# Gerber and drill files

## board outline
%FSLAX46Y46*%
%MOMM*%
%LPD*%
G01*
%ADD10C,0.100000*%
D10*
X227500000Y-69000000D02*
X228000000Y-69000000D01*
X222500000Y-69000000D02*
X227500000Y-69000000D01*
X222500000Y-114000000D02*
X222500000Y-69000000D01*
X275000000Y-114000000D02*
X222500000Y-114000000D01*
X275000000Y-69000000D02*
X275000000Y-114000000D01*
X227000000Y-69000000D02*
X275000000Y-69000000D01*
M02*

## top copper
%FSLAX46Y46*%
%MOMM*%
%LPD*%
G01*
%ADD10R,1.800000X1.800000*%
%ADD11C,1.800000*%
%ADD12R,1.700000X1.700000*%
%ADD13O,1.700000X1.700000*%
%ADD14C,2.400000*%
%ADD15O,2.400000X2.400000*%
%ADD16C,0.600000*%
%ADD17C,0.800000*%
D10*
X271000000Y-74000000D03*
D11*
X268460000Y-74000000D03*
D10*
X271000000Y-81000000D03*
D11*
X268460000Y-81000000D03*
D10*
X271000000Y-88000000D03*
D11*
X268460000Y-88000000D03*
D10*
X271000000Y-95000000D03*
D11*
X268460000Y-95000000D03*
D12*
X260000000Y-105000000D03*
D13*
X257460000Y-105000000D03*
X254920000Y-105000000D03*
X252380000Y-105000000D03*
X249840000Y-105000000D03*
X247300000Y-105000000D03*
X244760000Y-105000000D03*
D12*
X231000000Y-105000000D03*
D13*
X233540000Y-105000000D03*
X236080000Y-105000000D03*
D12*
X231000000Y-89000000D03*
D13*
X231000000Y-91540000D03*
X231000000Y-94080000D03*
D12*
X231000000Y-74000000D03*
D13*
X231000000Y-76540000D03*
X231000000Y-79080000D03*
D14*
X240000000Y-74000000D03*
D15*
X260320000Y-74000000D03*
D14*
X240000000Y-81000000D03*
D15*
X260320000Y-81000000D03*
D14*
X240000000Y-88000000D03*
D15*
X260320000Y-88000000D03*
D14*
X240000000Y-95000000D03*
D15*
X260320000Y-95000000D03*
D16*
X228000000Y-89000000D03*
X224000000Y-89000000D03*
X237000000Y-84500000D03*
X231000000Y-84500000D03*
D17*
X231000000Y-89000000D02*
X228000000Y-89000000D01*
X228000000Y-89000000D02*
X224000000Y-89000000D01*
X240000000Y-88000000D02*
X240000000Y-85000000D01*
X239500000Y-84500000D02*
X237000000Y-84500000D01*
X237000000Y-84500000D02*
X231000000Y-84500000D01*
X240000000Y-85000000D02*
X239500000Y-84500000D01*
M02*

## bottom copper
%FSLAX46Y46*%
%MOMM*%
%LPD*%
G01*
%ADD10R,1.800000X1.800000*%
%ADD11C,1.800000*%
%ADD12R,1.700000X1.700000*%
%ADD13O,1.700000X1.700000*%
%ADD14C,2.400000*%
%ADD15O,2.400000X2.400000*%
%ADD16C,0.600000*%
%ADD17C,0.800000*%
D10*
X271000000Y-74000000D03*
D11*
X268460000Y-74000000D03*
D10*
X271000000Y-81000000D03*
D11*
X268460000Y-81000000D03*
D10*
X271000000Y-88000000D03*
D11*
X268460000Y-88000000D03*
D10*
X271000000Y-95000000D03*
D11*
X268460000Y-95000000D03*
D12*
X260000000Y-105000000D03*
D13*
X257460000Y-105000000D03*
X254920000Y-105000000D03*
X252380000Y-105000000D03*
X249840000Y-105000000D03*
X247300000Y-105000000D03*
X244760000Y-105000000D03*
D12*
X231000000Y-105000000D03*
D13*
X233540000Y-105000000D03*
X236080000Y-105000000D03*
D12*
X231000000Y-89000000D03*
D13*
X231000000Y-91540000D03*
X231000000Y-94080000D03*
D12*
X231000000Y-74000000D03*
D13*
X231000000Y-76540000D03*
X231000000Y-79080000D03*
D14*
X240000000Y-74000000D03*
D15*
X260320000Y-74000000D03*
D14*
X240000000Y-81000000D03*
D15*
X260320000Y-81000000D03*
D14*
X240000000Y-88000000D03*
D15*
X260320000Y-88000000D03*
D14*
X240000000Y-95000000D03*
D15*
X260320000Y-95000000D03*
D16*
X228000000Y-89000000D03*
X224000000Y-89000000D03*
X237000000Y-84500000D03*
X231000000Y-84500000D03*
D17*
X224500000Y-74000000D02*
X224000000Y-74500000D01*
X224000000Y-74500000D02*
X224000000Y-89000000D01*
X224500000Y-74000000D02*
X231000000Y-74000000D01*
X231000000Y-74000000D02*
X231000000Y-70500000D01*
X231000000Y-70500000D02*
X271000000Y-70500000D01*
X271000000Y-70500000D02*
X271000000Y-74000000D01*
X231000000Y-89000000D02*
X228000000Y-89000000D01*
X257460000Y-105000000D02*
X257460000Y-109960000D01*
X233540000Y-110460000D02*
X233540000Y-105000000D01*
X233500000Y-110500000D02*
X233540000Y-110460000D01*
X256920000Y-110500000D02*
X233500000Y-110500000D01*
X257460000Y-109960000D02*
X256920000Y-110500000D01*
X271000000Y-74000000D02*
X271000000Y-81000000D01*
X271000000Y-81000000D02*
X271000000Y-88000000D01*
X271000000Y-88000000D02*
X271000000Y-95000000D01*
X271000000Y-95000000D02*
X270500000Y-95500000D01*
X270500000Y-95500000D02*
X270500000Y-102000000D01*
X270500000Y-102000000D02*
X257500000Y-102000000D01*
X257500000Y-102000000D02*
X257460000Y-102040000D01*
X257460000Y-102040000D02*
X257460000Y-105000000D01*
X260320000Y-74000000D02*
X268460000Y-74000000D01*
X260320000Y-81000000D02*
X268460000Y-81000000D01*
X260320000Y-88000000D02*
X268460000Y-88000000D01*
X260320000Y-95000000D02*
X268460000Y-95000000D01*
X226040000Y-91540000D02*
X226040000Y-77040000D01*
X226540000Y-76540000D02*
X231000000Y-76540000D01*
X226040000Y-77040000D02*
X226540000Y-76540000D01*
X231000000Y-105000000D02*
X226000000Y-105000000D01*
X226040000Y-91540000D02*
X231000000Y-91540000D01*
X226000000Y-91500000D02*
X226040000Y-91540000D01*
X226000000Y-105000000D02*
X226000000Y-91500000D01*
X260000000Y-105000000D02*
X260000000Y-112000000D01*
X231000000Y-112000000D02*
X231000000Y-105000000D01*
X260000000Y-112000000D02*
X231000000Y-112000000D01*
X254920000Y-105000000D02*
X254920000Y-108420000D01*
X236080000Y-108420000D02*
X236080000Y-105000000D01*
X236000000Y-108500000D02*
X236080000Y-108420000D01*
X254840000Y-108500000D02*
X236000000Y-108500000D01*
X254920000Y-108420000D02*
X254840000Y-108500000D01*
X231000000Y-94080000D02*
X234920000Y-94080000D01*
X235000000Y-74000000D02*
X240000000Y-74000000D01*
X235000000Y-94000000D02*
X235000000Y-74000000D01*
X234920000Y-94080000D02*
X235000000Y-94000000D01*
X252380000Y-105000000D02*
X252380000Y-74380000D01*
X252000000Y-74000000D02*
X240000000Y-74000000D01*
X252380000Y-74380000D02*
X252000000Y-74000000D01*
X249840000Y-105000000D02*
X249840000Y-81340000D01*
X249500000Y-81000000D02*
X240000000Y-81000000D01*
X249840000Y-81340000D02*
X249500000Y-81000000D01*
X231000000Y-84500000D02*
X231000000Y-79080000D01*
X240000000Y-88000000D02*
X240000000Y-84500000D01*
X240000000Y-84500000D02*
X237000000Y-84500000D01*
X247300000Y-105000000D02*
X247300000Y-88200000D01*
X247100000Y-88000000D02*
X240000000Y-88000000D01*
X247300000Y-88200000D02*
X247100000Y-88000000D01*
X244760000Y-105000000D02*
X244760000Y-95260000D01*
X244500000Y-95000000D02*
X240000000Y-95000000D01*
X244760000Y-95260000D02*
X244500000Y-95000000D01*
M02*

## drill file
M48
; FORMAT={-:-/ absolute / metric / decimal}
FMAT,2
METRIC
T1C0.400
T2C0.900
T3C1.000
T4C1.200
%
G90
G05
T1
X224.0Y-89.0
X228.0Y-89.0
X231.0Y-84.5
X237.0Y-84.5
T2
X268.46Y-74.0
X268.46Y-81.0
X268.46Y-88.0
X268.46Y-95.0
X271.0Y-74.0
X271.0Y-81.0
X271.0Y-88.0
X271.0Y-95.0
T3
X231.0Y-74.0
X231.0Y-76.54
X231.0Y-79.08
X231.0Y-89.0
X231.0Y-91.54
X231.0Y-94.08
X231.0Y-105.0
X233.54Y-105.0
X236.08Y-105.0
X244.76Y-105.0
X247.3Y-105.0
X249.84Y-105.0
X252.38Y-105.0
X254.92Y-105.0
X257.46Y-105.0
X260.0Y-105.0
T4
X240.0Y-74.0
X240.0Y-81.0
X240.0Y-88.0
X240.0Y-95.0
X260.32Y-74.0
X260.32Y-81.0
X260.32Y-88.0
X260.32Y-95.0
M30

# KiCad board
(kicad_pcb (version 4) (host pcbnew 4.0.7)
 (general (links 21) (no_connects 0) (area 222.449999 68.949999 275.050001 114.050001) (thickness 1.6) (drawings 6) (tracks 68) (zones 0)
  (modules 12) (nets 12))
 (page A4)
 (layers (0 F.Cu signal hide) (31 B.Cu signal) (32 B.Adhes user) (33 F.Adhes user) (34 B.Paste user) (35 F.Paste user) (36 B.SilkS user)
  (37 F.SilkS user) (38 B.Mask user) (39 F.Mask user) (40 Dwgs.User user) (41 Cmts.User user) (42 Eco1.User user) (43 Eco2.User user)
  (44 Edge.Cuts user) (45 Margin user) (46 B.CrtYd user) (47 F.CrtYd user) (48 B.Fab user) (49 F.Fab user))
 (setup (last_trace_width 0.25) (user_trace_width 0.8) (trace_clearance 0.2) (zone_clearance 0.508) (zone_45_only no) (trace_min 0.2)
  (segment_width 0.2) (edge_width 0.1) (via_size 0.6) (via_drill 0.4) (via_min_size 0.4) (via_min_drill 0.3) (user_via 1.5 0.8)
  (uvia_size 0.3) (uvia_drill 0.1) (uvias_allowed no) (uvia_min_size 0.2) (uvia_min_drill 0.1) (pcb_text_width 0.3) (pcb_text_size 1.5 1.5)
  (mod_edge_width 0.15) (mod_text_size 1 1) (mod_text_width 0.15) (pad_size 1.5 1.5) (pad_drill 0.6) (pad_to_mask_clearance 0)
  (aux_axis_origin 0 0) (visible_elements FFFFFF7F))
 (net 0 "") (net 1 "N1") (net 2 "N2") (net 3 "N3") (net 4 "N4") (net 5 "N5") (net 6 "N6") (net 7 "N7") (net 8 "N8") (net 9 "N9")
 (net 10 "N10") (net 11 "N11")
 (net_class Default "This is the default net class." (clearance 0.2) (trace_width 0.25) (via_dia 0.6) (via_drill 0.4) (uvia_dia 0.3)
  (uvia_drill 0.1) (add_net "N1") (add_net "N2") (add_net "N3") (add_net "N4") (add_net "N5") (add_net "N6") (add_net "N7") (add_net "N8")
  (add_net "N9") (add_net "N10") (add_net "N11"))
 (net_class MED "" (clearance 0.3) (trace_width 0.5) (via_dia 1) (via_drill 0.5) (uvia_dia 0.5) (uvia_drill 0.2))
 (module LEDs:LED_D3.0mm (layer F.Cu) (at 271 74 180)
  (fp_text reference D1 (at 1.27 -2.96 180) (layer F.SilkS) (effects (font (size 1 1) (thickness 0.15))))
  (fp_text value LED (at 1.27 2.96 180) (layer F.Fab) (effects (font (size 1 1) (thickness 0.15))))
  (pad 1 thru_hole rect (at 0 0 180) (size 1.8 1.8) (drill 0.9) (layers *.Cu *.Mask) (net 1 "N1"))
  (pad 2 thru_hole circle (at 2.54 0 180) (size 1.8 1.8) (drill 0.9) (layers *.Cu *.Mask) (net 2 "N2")))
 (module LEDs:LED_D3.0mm (layer F.Cu) (at 271 81 180)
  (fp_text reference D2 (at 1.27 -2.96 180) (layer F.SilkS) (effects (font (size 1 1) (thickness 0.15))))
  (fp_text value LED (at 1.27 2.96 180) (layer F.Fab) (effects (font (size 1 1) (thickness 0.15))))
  (pad 1 thru_hole rect (at 0 0 180) (size 1.8 1.8) (drill 0.9) (layers *.Cu *.Mask) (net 1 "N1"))
  (pad 2 thru_hole circle (at 2.54 0 180) (size 1.8 1.8) (drill 0.9) (layers *.Cu *.Mask) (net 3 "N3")))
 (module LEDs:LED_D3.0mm (layer F.Cu) (at 271 88 180)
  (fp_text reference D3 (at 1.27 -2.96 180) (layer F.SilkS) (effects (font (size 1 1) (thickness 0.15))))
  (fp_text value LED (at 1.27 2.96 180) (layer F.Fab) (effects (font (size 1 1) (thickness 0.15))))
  (pad 1 thru_hole rect (at 0 0 180) (size 1.8 1.8) (drill 0.9) (layers *.Cu *.Mask) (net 1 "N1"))
  (pad 2 thru_hole circle (at 2.54 0 180) (size 1.8 1.8) (drill 0.9) (layers *.Cu *.Mask) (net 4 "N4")))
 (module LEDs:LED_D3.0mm (layer F.Cu) (at 271 95 180)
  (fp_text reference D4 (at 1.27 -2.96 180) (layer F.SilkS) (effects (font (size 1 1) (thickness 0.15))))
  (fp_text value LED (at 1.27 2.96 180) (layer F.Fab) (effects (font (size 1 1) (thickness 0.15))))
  (pad 1 thru_hole rect (at 0 0 180) (size 1.8 1.8) (drill 0.9) (layers *.Cu *.Mask) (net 1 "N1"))
  (pad 2 thru_hole circle (at 2.54 0 180) (size 1.8 1.8) (drill 0.9) (layers *.Cu *.Mask) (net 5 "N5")))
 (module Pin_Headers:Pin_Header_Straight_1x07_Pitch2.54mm (layer F.Cu) (at 260 105 270)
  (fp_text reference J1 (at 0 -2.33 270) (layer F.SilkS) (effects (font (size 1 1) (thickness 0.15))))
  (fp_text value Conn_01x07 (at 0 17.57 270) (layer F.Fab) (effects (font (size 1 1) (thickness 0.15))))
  (pad 1 thru_hole rect (at 0 0 270) (size 1.7 1.7) (drill 1) (layers *.Cu *.Mask) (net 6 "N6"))
  (pad 2 thru_hole oval (at 0 2.54 270) (size 1.7 1.7) (drill 1) (layers *.Cu *.Mask) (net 1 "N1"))
  (pad 3 thru_hole oval (at 0 5.08 270) (size 1.7 1.7) (drill 1) (layers *.Cu *.Mask) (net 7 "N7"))
  (pad 4 thru_hole oval (at 0 7.62 270) (size 1.7 1.7) (drill 1) (layers *.Cu *.Mask) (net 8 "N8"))
  (pad 5 thru_hole oval (at 0 10.16 270) (size 1.7 1.7) (drill 1) (layers *.Cu *.Mask) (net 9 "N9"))
  (pad 6 thru_hole oval (at 0 12.7 270) (size 1.7 1.7) (drill 1) (layers *.Cu *.Mask) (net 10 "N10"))
  (pad 7 thru_hole oval (at 0 15.24 270) (size 1.7 1.7) (drill 1) (layers *.Cu *.Mask) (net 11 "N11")))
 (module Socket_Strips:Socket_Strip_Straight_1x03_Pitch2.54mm (layer F.Cu) (at 231 105 90)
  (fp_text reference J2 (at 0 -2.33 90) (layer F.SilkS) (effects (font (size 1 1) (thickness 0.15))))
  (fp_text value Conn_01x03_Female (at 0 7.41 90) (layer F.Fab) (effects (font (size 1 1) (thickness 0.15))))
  (pad 1 thru_hole rect (at 0 0 90) (size 1.7 1.7) (drill 1) (layers *.Cu *.Mask) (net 6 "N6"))
  (pad 2 thru_hole oval (at 0 2.54 90) (size 1.7 1.7) (drill 1) (layers *.Cu *.Mask) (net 1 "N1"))
  (pad 3 thru_hole oval (at 0 5.08 90) (size 1.7 1.7) (drill 1) (layers *.Cu *.Mask) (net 7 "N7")))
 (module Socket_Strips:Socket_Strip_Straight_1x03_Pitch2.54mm (layer F.Cu) (at 231 89)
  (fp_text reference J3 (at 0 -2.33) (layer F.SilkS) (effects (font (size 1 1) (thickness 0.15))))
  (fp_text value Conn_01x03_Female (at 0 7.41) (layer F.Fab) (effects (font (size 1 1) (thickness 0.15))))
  (pad 1 thru_hole rect (at 0 0) (size 1.7 1.7) (drill 1) (layers *.Cu *.Mask) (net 1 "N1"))
  (pad 2 thru_hole oval (at 0 2.54) (size 1.7 1.7) (drill 1) (layers *.Cu *.Mask) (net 6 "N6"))
  (pad 3 thru_hole oval (at 0 5.08) (size 1.7 1.7) (drill 1) (layers *.Cu *.Mask) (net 8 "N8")))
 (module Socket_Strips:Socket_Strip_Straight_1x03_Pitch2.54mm (layer F.Cu) (at 231 74)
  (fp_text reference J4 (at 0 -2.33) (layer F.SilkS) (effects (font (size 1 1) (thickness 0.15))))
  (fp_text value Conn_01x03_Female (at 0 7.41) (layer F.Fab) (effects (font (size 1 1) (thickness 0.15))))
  (pad 1 thru_hole rect (at 0 0) (size 1.7 1.7) (drill 1) (layers *.Cu *.Mask) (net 1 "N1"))
  (pad 2 thru_hole oval (at 0 2.54) (size 1.7 1.7) (drill 1) (layers *.Cu *.Mask) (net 6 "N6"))
  (pad 3 thru_hole oval (at 0 5.08) (size 1.7 1.7) (drill 1) (layers *.Cu *.Mask) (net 10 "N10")))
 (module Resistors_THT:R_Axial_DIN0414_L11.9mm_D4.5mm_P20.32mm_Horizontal (layer F.Cu) (at 240 74)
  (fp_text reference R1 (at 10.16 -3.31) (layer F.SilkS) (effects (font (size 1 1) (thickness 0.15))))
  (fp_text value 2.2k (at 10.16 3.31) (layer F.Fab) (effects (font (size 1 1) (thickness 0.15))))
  (pad 1 thru_hole circle (at 0 0) (size 2.4 2.4) (drill 1.2) (layers *.Cu *.Mask) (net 8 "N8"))
  (pad 2 thru_hole oval (at 20.32 0) (size 2.4 2.4) (drill 1.2) (layers *.Cu *.Mask) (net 2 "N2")))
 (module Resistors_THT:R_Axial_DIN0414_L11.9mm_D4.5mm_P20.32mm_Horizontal (layer F.Cu) (at 240 81)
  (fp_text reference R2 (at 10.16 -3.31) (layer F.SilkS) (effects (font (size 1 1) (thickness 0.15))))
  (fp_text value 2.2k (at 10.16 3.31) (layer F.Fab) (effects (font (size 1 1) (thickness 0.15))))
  (pad 1 thru_hole circle (at 0 0) (size 2.4 2.4) (drill 1.2) (layers *.Cu *.Mask) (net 9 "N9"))
  (pad 2 thru_hole oval (at 20.32 0) (size 2.4 2.4) (drill 1.2) (layers *.Cu *.Mask) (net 3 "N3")))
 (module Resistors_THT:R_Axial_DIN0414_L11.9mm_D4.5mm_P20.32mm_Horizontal (layer F.Cu) (at 240 88)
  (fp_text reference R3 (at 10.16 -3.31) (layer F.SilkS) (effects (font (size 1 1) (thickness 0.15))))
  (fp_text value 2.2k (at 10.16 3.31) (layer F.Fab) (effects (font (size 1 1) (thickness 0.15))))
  (pad 1 thru_hole circle (at 0 0) (size 2.4 2.4) (drill 1.2) (layers *.Cu *.Mask) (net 10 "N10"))
  (pad 2 thru_hole oval (at 20.32 0) (size 2.4 2.4) (drill 1.2) (layers *.Cu *.Mask) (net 4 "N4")))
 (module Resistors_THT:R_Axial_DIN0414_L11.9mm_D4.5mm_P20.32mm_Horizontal (layer F.Cu) (at 240 95)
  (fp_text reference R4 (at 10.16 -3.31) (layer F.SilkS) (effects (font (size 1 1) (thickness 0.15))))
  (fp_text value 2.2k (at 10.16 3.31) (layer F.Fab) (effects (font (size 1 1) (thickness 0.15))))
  (pad 1 thru_hole circle (at 0 0) (size 2.4 2.4) (drill 1.2) (layers *.Cu *.Mask) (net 11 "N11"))
  (pad 2 thru_hole oval (at 20.32 0) (size 2.4 2.4) (drill 1.2) (layers *.Cu *.Mask) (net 5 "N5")))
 (gr_line (start 227.5 69) (end 228 69) (angle 90) (layer Edge.Cuts) (width 0.1))
 (gr_line (start 222.5 69) (end 227.5 69) (angle 90) (layer Edge.Cuts) (width 0.1))
 (gr_line (start 222.5 114) (end 222.5 69) (angle 90) (layer Edge.Cuts) (width 0.1))
 (gr_line (start 275 114) (end 222.5 114) (angle 90) (layer Edge.Cuts) (width 0.1))
 (gr_line (start 275 69) (end 275 114) (angle 90) (layer Edge.Cuts) (width 0.1))
 (gr_line (start 227 69) (end 275 69) (angle 90) (layer Edge.Cuts) (width 0.1))
 (via (at 228 89) (size 0.6) (drill 0.4) (layers F.Cu B.Cu) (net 1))
 (segment (start 231 89) (end 228 89) (width 0.8) (layer F.Cu) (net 1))
 (segment (start 228 89) (end 224 89) (width 0.8) (layer F.Cu) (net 1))
 (segment (start 224.5 74) (end 224 74.5) (width 0.8) (layer B.Cu) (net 1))
 (segment (start 224 74.5) (end 224 89) (width 0.8) (layer B.Cu) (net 1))
 (segment (start 224.5 74) (end 231 74) (width 0.8) (layer B.Cu) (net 1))
 (via (at 224 89) (size 0.6) (drill 0.4) (layers F.Cu B.Cu) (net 1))
 (segment (start 231 74) (end 231 70.5) (width 0.8) (layer B.Cu) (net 1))
 (segment (start 231 70.5) (end 271 70.5) (width 0.8) (layer B.Cu) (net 1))
 (segment (start 271 70.5) (end 271 74) (width 0.8) (layer B.Cu) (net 1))
 (segment (start 231 89) (end 228 89) (width 0.8) (layer B.Cu) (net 1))
 (segment (start 257.46 105) (end 257.46 109.96) (width 0.8) (layer B.Cu) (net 1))
 (segment (start 233.54 110.46) (end 233.54 105) (width 0.8) (layer B.Cu) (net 1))
 (segment (start 233.5 110.5) (end 233.54 110.46) (width 0.8) (layer B.Cu) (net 1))
 (segment (start 256.92 110.5) (end 233.5 110.5) (width 0.8) (layer B.Cu) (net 1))
 (segment (start 257.46 109.96) (end 256.92 110.5) (width 0.8) (layer B.Cu) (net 1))
 (segment (start 271 74) (end 271 81) (width 0.8) (layer B.Cu) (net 1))
 (segment (start 271 81) (end 271 88) (width 0.8) (layer B.Cu) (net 1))
 (segment (start 271 88) (end 271 95) (width 0.8) (layer B.Cu) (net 1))
 (segment (start 271 95) (end 270.5 95.5) (width 0.8) (layer B.Cu) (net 1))
 (segment (start 270.5 95.5) (end 270.5 102) (width 0.8) (layer B.Cu) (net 1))
 (segment (start 270.5 102) (end 257.5 102) (width 0.8) (layer B.Cu) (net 1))
 (segment (start 257.5 102) (end 257.46 102.04) (width 0.8) (layer B.Cu) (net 1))
 (segment (start 257.46 102.04) (end 257.46 105) (width 0.8) (layer B.Cu) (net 1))
 (segment (start 260.32 74) (end 268.46 74) (width 0.8) (layer B.Cu) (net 2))
 (segment (start 260.32 81) (end 268.46 81) (width 0.8) (layer B.Cu) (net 3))
 (segment (start 260.32 88) (end 268.46 88) (width 0.8) (layer B.Cu) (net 4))
 (segment (start 260.32 95) (end 268.46 95) (width 0.8) (layer B.Cu) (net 5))
 (segment (start 226.04 91.54) (end 226.04 77.04) (width 0.8) (layer B.Cu) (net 6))
 (segment (start 226.54 76.54) (end 231 76.54) (width 0.8) (layer B.Cu) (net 6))
 (segment (start 226.04 77.04) (end 226.54 76.54) (width 0.8) (layer B.Cu) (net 6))
 (segment (start 231 105) (end 226 105) (width 0.8) (layer B.Cu) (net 6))
 (segment (start 226.04 91.54) (end 231 91.54) (width 0.8) (layer B.Cu) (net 6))
 (segment (start 226 91.5) (end 226.04 91.54) (width 0.8) (layer B.Cu) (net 6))
 (segment (start 226 105) (end 226 91.5) (width 0.8) (layer B.Cu) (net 6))
 (segment (start 260 105) (end 260 112) (width 0.8) (layer B.Cu) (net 6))
 (segment (start 231 112) (end 231 105) (width 0.8) (layer B.Cu) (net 6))
 (segment (start 260 112) (end 231 112) (width 0.8) (layer B.Cu) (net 6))
 (segment (start 254.92 105) (end 254.92 108.42) (width 0.8) (layer B.Cu) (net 7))
 (segment (start 236.08 108.42) (end 236.08 105) (width 0.8) (layer B.Cu) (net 7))
 (segment (start 236 108.5) (end 236.08 108.42) (width 0.8) (layer B.Cu) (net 7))
 (segment (start 254.84 108.5) (end 236 108.5) (width 0.8) (layer B.Cu) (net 7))
 (segment (start 254.92 108.42) (end 254.84 108.5) (width 0.8) (layer B.Cu) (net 7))
 (segment (start 231 94.08) (end 234.92 94.08) (width 0.8) (layer B.Cu) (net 8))
 (segment (start 235 74) (end 240 74) (width 0.8) (layer B.Cu) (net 8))
 (segment (start 235 94) (end 235 74) (width 0.8) (layer B.Cu) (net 8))
 (segment (start 234.92 94.08) (end 235 94) (width 0.8) (layer B.Cu) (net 8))
 (segment (start 252.38 105) (end 252.38 74.38) (width 0.8) (layer B.Cu) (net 8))
 (segment (start 252 74) (end 240 74) (width 0.8) (layer B.Cu) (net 8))
 (segment (start 252.38 74.38) (end 252 74) (width 0.8) (layer B.Cu) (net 8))
 (segment (start 249.84 105) (end 249.84 81.34) (width 0.8) (layer B.Cu) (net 9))
 (segment (start 249.5 81) (end 240 81) (width 0.8) (layer B.Cu) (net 9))
 (segment (start 249.84 81.34) (end 249.5 81) (width 0.8) (layer B.Cu) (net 9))
 (via (at 237 84.5) (size 0.6) (drill 0.4) (layers F.Cu B.Cu) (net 10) (status 1000000))
 (segment (start 240 88) (end 240 85) (width 0.8) (layer F.Cu) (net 10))
 (segment (start 231 84.5) (end 231 79.08) (width 0.8) (layer B.Cu) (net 10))
 (via (at 231 84.5) (size 0.6) (drill 0.4) (layers F.Cu B.Cu) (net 10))
 (segment (start 239.5 84.5) (end 237 84.5) (width 0.8) (layer F.Cu) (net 10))
 (segment (start 237 84.5) (end 231 84.5) (width 0.8) (layer F.Cu) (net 10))
 (segment (start 240 85) (end 239.5 84.5) (width 0.8) (layer F.Cu) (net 10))
 (segment (start 240 88) (end 240 84.5) (width 0.8) (layer B.Cu) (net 10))
 (segment (start 240 84.5) (end 237 84.5) (width 0.8) (layer B.Cu) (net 10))
 (segment (start 247.3 105) (end 247.3 88.2) (width 0.8) (layer B.Cu) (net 10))
 (segment (start 247.1 88) (end 240 88) (width 0.8) (layer B.Cu) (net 10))
 (segment (start 247.3 88.2) (end 247.1 88) (width 0.8) (layer B.Cu) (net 10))
 (segment (start 244.76 105) (end 244.76 95.26) (width 0.8) (layer B.Cu) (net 11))
 (segment (start 244.5 95) (end 240 95) (width 0.8) (layer B.Cu) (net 11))
 (segment (start 244.76 95.26) (end 244.5 95) (width 0.8) (layer B.Cu) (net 11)))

